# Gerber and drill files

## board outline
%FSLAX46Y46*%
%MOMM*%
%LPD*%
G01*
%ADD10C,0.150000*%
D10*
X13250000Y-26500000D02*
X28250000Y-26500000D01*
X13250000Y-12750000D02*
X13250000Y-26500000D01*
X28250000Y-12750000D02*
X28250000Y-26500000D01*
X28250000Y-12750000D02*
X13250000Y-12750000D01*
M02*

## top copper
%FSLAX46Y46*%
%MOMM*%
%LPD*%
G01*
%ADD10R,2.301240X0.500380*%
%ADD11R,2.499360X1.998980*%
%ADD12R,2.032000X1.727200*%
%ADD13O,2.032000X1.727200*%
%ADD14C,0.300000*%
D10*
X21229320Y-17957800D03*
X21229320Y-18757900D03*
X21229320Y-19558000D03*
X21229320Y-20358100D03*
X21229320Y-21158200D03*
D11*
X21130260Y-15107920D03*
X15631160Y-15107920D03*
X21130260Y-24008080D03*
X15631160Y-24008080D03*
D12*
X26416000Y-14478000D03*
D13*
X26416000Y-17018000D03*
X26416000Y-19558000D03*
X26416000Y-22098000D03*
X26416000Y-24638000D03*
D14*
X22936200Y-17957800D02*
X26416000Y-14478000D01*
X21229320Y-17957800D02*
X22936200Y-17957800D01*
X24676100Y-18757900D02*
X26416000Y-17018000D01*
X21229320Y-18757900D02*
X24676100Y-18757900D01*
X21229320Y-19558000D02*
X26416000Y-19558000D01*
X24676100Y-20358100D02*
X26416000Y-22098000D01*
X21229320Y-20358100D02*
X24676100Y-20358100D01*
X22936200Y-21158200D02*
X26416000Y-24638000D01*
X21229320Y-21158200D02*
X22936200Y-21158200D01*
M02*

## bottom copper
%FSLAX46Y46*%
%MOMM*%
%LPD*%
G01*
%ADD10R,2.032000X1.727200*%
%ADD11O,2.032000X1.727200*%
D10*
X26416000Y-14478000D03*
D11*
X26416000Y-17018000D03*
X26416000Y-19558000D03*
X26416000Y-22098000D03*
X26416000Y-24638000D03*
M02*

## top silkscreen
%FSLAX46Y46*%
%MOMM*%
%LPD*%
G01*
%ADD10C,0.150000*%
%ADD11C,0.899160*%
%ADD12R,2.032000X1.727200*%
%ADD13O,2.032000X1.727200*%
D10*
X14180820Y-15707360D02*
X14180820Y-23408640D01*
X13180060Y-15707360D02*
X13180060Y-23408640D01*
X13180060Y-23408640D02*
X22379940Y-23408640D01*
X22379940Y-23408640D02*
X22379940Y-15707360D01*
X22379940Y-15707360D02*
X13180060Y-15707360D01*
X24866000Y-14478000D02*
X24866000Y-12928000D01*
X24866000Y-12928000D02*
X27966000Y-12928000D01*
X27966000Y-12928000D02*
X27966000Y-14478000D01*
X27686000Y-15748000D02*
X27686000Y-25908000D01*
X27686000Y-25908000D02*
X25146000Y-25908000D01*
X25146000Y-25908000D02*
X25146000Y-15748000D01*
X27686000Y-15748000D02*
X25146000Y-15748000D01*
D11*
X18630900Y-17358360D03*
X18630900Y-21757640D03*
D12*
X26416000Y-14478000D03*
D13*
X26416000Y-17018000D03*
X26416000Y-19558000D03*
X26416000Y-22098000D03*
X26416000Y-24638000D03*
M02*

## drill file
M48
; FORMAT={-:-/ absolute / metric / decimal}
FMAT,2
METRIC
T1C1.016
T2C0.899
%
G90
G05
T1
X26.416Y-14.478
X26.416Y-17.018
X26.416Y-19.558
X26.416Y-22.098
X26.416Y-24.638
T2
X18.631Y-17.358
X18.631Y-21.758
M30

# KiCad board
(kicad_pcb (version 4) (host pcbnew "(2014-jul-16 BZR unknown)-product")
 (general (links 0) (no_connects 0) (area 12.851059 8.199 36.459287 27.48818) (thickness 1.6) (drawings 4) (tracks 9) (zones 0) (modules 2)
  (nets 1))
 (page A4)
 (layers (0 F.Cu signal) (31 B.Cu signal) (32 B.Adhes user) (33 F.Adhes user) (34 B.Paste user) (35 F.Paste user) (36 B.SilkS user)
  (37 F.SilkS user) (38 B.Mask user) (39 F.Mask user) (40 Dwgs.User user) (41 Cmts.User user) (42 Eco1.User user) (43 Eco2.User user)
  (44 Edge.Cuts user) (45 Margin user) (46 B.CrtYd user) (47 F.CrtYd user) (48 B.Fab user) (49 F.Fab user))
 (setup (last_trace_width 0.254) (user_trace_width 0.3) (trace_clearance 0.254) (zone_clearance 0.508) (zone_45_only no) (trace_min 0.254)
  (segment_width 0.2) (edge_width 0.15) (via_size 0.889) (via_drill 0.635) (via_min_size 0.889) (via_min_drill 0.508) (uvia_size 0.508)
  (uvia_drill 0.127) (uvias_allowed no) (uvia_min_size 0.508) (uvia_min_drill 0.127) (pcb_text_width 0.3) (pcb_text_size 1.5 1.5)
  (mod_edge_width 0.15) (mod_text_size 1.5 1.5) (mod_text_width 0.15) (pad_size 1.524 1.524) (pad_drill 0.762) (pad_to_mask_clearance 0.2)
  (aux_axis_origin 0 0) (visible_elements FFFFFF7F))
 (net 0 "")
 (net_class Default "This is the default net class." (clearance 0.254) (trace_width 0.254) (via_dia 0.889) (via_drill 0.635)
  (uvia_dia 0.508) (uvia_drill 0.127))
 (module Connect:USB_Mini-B (layer F.Cu) (at 17.78 19.558)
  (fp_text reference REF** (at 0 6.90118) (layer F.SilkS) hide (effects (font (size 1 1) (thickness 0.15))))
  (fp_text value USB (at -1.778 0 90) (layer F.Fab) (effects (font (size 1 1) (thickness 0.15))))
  (fp_line (start -3.59918 -3.85064) (end -3.59918 3.85064) (layer F.SilkS) (width 0.15))
  (fp_line (start -4.59994 -3.85064) (end -4.59994 3.85064) (layer F.SilkS) (width 0.15))
  (fp_line (start -4.59994 3.85064) (end 4.59994 3.85064) (layer F.SilkS) (width 0.15))
  (fp_line (start 4.59994 3.85064) (end 4.59994 -3.85064) (layer F.SilkS) (width 0.15))
  (fp_line (start 4.59994 -3.85064) (end -4.59994 -3.85064) (layer F.SilkS) (width 0.15))
  (pad 1 smd rect (at 3.44932 -1.6002) (size 2.30124 0.50038) (layers F.Cu F.Paste F.Mask))
  (pad 2 smd rect (at 3.44932 -0.8001) (size 2.30124 0.50038) (layers F.Cu F.Paste F.Mask))
  (pad 3 smd rect (at 3.44932 0) (size 2.30124 0.50038) (layers F.Cu F.Paste F.Mask))
  (pad 4 smd rect (at 3.44932 0.8001) (size 2.30124 0.50038) (layers F.Cu F.Paste F.Mask))
  (pad 5 smd rect (at 3.44932 1.6002) (size 2.30124 0.50038) (layers F.Cu F.Paste F.Mask))
  (pad 6 smd rect (at 3.35026 -4.45008) (size 2.49936 1.99898) (layers F.Cu F.Paste F.Mask))
  (pad 7 smd rect (at -2.14884 -4.45008) (size 2.49936 1.99898) (layers F.Cu F.Paste F.Mask))
  (pad 8 smd rect (at 3.35026 4.45008) (size 2.49936 1.99898) (layers F.Cu F.Paste F.Mask))
  (pad 9 smd rect (at -2.14884 4.45008) (size 2.49936 1.99898) (layers F.Cu F.Paste F.Mask))
  (pad "" np_thru_hole circle (at 0.8509 -2.19964) (size 0.89916 0.89916) (drill 0.89916) (layers *.Cu *.Mask F.SilkS))
  (pad 2 np_thru_hole circle (at 0.8509 2.19964) (size 0.89916 0.89916) (drill 0.89916) (layers *.Cu *.Mask F.SilkS)))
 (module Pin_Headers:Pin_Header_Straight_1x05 (layer F.Cu) (at 26.416 14.478)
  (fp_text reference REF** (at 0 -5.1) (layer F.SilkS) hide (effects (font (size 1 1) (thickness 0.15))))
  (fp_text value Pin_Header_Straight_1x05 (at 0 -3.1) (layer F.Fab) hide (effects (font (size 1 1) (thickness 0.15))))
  (fp_line (start -1.55 0) (end -1.55 -1.55) (layer F.SilkS) (width 0.15))
  (fp_line (start -1.55 -1.55) (end 1.55 -1.55) (layer F.SilkS) (width 0.15))
  (fp_line (start 1.55 -1.55) (end 1.55 0) (layer F.SilkS) (width 0.15))
  (fp_line (start 1.27 1.27) (end 1.27 11.43) (layer F.SilkS) (width 0.15))
  (fp_line (start 1.27 11.43) (end -1.27 11.43) (layer F.SilkS) (width 0.15))
  (fp_line (start -1.27 11.43) (end -1.27 1.27) (layer F.SilkS) (width 0.15))
  (fp_line (start 1.27 1.27) (end -1.27 1.27) (layer F.SilkS) (width 0.15))
  (pad 1 thru_hole rect (at 0 0) (size 2.032 1.7272) (drill 1.016) (layers *.Cu *.Mask F.SilkS))
  (pad 2 thru_hole oval (at 0 2.54) (size 2.032 1.7272) (drill 1.016) (layers *.Cu *.Mask F.SilkS))
  (pad 3 thru_hole oval (at 0 5.08) (size 2.032 1.7272) (drill 1.016) (layers *.Cu *.Mask F.SilkS))
  (pad 4 thru_hole oval (at 0 7.62) (size 2.032 1.7272) (drill 1.016) (layers *.Cu *.Mask F.SilkS))
  (pad 5 thru_hole oval (at 0 10.16) (size 2.032 1.7272) (drill 1.016) (layers *.Cu *.Mask F.SilkS)))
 (gr_line (start 13.25 26.5) (end 28.25 26.5) (angle 90) (layer Edge.Cuts) (width 0.15))
 (gr_line (start 13.25 12.75) (end 13.25 26.5) (angle 90) (layer Edge.Cuts) (width 0.15))
 (gr_line (start 28.25 12.75) (end 28.25 26.5) (angle 90) (layer Edge.Cuts) (width 0.15))
 (gr_line (start 28.25 12.75) (end 13.25 12.75) (angle 90) (layer Edge.Cuts) (width 0.15))
 (segment (start 22.9362 17.9578) (end 26.416 14.478) (width 0.3) (layer F.Cu) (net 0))
 (segment (start 21.22932 17.9578) (end 22.9362 17.9578) (width 0.3) (layer F.Cu) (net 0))
 (segment (start 24.6761 18.7579) (end 26.416 17.018) (width 0.3) (layer F.Cu) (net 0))
 (segment (start 21.22932 18.7579) (end 24.6761 18.7579) (width 0.3) (layer F.Cu) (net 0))
 (segment (start 21.22932 19.558) (end 26.416 19.558) (width 0.3) (layer F.Cu) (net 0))
 (segment (start 24.6761 20.3581) (end 26.416 22.098) (width 0.3) (layer F.Cu) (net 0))
 (segment (start 21.22932 20.3581) (end 24.6761 20.3581) (width 0.3) (layer F.Cu) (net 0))
 (segment (start 22.9362 21.1582) (end 26.416 24.638) (width 0.3) (layer F.Cu) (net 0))
 (segment (start 21.22932 21.1582) (end 22.9362 21.1582) (width 0.3) (layer F.Cu) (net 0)))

